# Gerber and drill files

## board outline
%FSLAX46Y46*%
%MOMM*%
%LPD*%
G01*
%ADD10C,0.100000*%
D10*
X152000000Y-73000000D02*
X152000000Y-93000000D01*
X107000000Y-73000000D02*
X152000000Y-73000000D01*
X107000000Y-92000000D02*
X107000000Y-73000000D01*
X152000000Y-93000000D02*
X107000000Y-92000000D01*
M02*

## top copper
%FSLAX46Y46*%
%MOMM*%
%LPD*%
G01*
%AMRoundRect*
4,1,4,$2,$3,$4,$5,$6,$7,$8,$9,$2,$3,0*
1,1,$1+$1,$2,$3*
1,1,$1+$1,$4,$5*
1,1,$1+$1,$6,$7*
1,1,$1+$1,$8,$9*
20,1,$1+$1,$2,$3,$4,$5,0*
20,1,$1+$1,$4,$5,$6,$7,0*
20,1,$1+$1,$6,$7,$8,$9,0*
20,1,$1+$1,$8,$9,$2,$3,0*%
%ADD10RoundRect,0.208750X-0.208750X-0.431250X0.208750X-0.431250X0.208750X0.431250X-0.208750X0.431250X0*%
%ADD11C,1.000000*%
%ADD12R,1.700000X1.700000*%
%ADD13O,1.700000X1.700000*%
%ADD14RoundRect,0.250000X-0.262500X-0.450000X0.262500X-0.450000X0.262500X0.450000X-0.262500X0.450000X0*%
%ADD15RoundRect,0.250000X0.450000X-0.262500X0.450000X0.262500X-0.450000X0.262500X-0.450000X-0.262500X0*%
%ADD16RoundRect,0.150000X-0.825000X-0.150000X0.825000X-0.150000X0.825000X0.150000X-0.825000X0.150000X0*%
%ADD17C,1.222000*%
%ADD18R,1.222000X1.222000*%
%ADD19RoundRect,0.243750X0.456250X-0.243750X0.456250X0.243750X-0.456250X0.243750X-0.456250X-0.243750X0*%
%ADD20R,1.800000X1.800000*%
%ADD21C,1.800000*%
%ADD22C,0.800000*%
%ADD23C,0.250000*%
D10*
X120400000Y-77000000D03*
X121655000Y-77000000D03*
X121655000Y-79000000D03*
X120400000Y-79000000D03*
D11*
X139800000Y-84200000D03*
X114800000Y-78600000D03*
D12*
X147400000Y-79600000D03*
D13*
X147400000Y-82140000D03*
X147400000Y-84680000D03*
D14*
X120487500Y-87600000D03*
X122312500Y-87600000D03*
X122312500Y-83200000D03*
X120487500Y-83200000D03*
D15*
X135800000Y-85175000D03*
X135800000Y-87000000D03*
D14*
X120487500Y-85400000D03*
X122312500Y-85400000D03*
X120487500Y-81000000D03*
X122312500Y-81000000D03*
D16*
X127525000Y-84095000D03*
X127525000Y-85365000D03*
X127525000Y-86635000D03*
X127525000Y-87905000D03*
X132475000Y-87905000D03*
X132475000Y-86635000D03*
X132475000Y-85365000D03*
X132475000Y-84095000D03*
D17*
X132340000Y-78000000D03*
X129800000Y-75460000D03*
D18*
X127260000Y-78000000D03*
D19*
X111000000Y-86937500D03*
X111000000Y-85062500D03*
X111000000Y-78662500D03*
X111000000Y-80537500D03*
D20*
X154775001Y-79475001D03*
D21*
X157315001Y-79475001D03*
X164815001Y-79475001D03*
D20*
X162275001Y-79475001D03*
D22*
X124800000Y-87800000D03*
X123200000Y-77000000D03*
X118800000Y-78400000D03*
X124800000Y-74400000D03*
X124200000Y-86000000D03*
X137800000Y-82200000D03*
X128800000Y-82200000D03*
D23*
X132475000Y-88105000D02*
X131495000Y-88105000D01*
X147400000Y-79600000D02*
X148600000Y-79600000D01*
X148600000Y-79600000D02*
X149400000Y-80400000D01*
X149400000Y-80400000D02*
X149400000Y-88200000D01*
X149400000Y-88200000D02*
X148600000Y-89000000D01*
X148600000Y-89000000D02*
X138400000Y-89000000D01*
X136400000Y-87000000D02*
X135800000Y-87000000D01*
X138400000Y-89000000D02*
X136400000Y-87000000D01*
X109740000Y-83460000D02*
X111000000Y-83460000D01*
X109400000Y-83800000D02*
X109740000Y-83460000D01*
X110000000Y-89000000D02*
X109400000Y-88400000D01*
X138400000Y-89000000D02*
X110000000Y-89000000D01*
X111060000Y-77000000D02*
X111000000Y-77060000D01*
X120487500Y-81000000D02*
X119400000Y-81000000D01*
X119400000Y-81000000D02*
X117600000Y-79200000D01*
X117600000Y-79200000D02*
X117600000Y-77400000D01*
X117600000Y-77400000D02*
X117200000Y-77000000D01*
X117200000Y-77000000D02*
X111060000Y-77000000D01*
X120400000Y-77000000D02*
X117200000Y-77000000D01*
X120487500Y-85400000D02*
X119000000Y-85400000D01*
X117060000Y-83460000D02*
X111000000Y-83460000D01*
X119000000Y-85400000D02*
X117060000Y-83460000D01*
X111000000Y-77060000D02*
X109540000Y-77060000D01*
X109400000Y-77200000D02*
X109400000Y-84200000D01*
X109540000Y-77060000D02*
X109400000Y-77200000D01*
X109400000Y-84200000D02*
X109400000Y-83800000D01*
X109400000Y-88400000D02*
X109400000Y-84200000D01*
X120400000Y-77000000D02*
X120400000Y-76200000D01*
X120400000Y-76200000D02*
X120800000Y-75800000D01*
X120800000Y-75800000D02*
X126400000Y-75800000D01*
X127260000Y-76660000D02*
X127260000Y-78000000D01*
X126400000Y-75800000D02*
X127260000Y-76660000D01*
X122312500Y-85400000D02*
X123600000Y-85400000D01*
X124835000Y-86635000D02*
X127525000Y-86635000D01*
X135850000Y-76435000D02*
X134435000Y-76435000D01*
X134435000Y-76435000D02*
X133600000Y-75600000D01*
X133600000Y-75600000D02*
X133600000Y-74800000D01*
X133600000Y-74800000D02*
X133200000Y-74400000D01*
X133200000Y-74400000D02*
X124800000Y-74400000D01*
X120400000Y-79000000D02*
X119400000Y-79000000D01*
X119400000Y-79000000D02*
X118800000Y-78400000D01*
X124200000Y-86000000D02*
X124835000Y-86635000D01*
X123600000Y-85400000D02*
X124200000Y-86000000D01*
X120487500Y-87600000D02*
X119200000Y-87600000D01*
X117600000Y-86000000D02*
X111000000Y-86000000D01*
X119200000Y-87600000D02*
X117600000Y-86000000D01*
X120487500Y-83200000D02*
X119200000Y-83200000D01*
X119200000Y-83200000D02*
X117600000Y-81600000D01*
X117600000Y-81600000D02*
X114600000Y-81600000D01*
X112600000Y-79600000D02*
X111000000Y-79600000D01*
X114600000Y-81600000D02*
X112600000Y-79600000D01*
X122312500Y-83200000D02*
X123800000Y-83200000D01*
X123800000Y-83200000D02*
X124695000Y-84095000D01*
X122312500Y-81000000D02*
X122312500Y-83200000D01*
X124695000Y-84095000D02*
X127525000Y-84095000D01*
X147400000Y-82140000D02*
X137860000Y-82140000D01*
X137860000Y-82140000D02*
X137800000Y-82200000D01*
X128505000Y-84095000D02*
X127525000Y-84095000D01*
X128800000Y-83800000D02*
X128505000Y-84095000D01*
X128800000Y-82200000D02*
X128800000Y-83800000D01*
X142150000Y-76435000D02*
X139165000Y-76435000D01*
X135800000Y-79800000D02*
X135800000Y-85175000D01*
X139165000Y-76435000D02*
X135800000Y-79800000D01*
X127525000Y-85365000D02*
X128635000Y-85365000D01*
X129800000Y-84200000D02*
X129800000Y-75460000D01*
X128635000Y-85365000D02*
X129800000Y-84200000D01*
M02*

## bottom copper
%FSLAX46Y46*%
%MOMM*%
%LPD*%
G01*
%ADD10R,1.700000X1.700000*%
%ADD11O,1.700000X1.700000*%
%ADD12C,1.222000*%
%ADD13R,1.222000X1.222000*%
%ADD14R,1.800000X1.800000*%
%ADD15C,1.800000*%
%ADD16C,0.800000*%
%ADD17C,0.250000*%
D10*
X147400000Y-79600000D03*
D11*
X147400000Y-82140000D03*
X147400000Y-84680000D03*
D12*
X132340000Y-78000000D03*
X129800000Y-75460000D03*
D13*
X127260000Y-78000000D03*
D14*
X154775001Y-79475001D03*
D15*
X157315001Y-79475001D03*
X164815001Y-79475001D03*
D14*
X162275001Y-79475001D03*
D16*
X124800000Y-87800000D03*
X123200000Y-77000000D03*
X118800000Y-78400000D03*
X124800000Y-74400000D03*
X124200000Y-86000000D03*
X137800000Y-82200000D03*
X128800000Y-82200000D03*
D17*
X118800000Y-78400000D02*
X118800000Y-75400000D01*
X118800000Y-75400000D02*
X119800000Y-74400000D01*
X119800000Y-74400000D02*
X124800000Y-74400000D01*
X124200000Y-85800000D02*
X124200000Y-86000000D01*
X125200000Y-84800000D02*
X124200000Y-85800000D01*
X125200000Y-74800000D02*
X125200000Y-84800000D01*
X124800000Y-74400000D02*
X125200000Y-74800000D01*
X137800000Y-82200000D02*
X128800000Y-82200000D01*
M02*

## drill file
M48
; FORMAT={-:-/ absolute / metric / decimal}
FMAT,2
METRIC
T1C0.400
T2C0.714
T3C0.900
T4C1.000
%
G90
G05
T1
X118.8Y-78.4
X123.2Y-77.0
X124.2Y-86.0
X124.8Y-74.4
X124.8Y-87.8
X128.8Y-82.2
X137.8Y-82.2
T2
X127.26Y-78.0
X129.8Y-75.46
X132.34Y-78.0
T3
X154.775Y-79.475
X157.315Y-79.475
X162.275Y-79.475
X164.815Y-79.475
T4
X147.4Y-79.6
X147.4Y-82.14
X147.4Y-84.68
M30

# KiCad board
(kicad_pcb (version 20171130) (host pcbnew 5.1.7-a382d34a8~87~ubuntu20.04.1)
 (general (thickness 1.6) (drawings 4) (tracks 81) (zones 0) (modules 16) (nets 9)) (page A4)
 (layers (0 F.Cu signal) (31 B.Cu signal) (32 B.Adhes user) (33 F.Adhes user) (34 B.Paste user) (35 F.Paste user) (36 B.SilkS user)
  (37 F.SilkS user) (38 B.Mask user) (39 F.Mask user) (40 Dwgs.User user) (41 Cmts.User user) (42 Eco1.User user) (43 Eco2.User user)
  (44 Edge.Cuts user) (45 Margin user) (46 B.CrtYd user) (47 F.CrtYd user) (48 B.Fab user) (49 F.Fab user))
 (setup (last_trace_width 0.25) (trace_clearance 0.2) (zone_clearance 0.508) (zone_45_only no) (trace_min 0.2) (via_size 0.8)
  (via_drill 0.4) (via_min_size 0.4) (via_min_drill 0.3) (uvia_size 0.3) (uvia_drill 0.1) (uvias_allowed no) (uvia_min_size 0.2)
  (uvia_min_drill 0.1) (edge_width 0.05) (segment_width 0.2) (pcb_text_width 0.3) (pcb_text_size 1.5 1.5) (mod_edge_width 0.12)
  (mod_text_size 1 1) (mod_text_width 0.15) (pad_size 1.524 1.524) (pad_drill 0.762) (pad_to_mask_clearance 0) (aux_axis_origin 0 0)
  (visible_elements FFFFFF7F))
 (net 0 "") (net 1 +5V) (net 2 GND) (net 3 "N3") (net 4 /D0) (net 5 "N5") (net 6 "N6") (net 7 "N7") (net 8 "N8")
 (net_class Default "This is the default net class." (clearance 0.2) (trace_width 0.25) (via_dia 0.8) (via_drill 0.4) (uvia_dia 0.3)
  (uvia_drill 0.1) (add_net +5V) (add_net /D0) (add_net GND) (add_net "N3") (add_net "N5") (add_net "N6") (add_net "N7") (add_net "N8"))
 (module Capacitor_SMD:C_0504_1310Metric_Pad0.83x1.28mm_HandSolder (layer F.Cu) (at 121.0275 77)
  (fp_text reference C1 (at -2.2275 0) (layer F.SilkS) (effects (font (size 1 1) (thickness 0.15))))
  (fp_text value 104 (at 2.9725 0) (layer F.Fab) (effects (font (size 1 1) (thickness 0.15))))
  (pad 1 smd roundrect (at -0.6275 0) (size 0.835 1.28) (layers F.Cu F.Paste F.Mask) (roundrect_rratio 0.25) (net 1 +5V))
  (pad 2 smd roundrect (at 0.6275 0) (size 0.835 1.28) (layers F.Cu F.Paste F.Mask) (roundrect_rratio 0.25) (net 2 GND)))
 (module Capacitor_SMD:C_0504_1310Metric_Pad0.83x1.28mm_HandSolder (layer F.Cu) (at 121.0275 79)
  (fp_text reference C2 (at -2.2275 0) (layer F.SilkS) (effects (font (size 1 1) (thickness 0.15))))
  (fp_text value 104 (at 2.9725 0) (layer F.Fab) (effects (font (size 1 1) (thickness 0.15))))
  (pad 2 smd roundrect (at 0.6275 0) (size 0.835 1.28) (layers F.Cu F.Paste F.Mask) (roundrect_rratio 0.25) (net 2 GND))
  (pad 1 smd roundrect (at -0.6275 0) (size 0.835 1.28) (layers F.Cu F.Paste F.Mask) (roundrect_rratio 0.25) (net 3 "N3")))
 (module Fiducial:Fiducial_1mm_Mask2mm (layer F.Cu) (at 139.8 84.2)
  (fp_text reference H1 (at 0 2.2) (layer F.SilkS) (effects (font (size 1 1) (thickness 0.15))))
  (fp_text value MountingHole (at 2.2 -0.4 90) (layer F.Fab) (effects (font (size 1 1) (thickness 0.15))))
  (pad "" smd circle (at 0 0) (size 1 1) (layers F.Cu F.Mask) (solder_mask_margin 0.5) (clearance 0.5)))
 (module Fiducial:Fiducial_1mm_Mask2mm (layer F.Cu) (at 114.8 78.6)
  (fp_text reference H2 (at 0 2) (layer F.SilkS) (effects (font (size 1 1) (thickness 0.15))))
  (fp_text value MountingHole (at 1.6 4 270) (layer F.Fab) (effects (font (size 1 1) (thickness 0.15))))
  (pad "" smd circle (at 0 0) (size 1 1) (layers F.Cu F.Mask) (solder_mask_margin 0.5) (clearance 0.5)))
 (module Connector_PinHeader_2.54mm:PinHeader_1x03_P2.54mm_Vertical (layer F.Cu) (at 147.4 79.6)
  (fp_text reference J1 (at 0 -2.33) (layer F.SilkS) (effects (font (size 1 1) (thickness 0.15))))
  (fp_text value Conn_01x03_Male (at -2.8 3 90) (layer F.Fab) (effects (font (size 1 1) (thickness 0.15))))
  (pad 1 thru_hole rect (at 0 0) (size 1.7 1.7) (drill 1) (layers *.Cu *.Mask) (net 1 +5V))
  (pad 2 thru_hole oval (at 0 2.54) (size 1.7 1.7) (drill 1) (layers *.Cu *.Mask) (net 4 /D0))
  (pad 3 thru_hole oval (at 0 5.08) (size 1.7 1.7) (drill 1) (layers *.Cu *.Mask) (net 2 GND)))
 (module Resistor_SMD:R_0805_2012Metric (layer F.Cu) (at 121.4 87.6)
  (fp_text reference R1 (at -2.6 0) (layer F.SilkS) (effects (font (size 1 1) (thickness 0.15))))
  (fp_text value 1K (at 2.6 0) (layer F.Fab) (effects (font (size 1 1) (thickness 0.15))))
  (pad 1 smd roundrect (at -0.9125 0) (size 1.025 1.4) (layers F.Cu F.Paste F.Mask) (roundrect_rratio 0.243902) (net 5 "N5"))
  (pad 2 smd roundrect (at 0.9125 0) (size 1.025 1.4) (layers F.Cu F.Paste F.Mask) (roundrect_rratio 0.243902) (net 2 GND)))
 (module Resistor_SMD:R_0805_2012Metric (layer F.Cu) (at 121.4 83.2)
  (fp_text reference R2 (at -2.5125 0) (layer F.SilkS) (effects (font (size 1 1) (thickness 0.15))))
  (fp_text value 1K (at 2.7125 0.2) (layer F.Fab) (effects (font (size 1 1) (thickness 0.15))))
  (pad 2 smd roundrect (at 0.9125 0) (size 1.025 1.4) (layers F.Cu F.Paste F.Mask) (roundrect_rratio 0.243902) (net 4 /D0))
  (pad 1 smd roundrect (at -0.9125 0) (size 1.025 1.4) (layers F.Cu F.Paste F.Mask) (roundrect_rratio 0.243902) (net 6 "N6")))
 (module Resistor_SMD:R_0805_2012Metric (layer F.Cu) (at 135.8 86.0875 90)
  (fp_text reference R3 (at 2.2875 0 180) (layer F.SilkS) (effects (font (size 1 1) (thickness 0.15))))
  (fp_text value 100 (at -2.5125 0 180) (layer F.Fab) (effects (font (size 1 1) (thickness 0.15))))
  (pad 2 smd roundrect (at 0.9125 0 90) (size 1.025 1.4) (layers F.Cu F.Paste F.Mask) (roundrect_rratio 0.243902) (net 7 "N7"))
  (pad 1 smd roundrect (at -0.9125 0 90) (size 1.025 1.4) (layers F.Cu F.Paste F.Mask) (roundrect_rratio 0.243902) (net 1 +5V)))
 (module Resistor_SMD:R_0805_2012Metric (layer F.Cu) (at 121.4 85.4)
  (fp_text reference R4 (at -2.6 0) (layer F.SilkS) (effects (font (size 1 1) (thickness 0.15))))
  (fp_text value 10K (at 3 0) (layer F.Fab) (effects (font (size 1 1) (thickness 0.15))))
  (pad 1 smd roundrect (at -0.9125 0) (size 1.025 1.4) (layers F.Cu F.Paste F.Mask) (roundrect_rratio 0.243902) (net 1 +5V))
  (pad 2 smd roundrect (at 0.9125 0) (size 1.025 1.4) (layers F.Cu F.Paste F.Mask) (roundrect_rratio 0.243902) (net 3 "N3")))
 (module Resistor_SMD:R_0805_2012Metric (layer F.Cu) (at 121.4 81)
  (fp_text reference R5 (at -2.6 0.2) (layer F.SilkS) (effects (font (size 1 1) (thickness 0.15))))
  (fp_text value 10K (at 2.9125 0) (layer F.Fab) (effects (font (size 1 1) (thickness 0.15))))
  (pad 1 smd roundrect (at -0.9125 0) (size 1.025 1.4) (layers F.Cu F.Paste F.Mask) (roundrect_rratio 0.243902) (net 1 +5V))
  (pad 2 smd roundrect (at 0.9125 0) (size 1.025 1.4) (layers F.Cu F.Paste F.Mask) (roundrect_rratio 0.243902) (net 4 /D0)))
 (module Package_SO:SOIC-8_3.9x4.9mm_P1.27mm (layer F.Cu) (at 130 86)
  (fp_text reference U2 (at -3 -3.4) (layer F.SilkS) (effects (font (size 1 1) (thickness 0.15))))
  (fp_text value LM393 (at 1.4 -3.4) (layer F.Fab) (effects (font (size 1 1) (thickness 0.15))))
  (pad 1 smd roundrect (at -2.475 -1.905) (size 1.95 0.6) (layers F.Cu F.Paste F.Mask) (roundrect_rratio 0.25) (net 4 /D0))
  (pad 2 smd roundrect (at -2.475 -0.635) (size 1.95 0.6) (layers F.Cu F.Paste F.Mask) (roundrect_rratio 0.25) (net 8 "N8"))
  (pad 3 smd roundrect (at -2.475 0.635) (size 1.95 0.6) (layers F.Cu F.Paste F.Mask) (roundrect_rratio 0.25) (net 3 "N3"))
  (pad 4 smd roundrect (at -2.475 1.905) (size 1.95 0.6) (layers F.Cu F.Paste F.Mask) (roundrect_rratio 0.25))
  (pad 5 smd roundrect (at 2.475 1.905) (size 1.95 0.6) (layers F.Cu F.Paste F.Mask) (roundrect_rratio 0.25))
  (pad 6 smd roundrect (at 2.475 0.635) (size 1.95 0.6) (layers F.Cu F.Paste F.Mask) (roundrect_rratio 0.25))
  (pad 7 smd roundrect (at 2.475 -0.635) (size 1.95 0.6) (layers F.Cu F.Paste F.Mask) (roundrect_rratio 0.25))
  (pad 8 smd roundrect (at 2.475 -1.905) (size 1.95 0.6) (layers F.Cu F.Paste F.Mask) (roundrect_rratio 0.25)))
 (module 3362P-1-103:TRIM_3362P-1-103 (layer F.Cu) (at 129.8 78)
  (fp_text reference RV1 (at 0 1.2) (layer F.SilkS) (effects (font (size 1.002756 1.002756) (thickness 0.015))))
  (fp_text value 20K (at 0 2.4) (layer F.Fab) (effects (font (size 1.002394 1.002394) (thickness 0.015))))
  (pad 3 thru_hole circle (at 2.54 0) (size 1.222 1.222) (drill 0.714) (layers *.Cu *.Mask) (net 2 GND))
  (pad 2 thru_hole circle (at 0 -2.54) (size 1.222 1.222) (drill 0.714) (layers *.Cu *.Mask) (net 8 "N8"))
  (pad 1 thru_hole rect (at -2.54 0) (size 1.222 1.222) (drill 0.714) (layers *.Cu *.Mask) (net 1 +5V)))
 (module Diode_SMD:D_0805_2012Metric (layer F.Cu) (at 111 86 90)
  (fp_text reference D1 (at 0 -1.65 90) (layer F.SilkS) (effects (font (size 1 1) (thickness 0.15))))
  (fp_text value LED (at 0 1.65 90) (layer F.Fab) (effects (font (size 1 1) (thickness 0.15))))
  (pad 1 smd roundrect (at -0.9375 0 90) (size 0.975 1.4) (layers F.Cu F.Paste F.Mask) (roundrect_rratio 0.25) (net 5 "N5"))
  (pad 2 smd roundrect (at 0.9375 0 90) (size 0.975 1.4) (layers F.Cu F.Paste F.Mask) (roundrect_rratio 0.25) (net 1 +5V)))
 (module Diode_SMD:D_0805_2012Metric (layer F.Cu) (at 111 79.6 90)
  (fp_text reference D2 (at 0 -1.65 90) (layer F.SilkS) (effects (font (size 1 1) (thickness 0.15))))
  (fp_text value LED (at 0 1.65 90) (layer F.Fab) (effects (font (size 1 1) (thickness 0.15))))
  (pad 2 smd roundrect (at 0.9375 0 90) (size 0.975 1.4) (layers F.Cu F.Paste F.Mask) (roundrect_rratio 0.25) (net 1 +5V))
  (pad 1 smd roundrect (at -0.9375 0 90) (size 0.975 1.4) (layers F.Cu F.Paste F.Mask) (roundrect_rratio 0.25) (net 6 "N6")))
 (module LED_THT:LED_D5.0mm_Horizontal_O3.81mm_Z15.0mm (layer F.Cu) (at 154.775001 79.475001)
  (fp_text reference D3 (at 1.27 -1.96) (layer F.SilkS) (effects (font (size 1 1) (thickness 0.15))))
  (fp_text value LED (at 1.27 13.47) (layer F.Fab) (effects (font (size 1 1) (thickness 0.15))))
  (pad 1 thru_hole rect (at 0 0) (size 1.8 1.8) (drill 0.9) (layers *.Cu *.Mask) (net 2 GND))
  (pad 2 thru_hole circle (at 2.54 0) (size 1.8 1.8) (drill 0.9) (layers *.Cu *.Mask) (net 7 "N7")))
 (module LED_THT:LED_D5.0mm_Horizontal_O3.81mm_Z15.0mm (layer F.Cu) (at 162.275001 79.475001)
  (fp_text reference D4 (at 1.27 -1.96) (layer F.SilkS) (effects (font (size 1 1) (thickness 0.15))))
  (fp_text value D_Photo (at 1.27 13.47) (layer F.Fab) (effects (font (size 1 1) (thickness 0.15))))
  (pad 2 thru_hole circle (at 2.54 0) (size 1.8 1.8) (drill 0.9) (layers *.Cu *.Mask) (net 3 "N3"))
  (pad 1 thru_hole rect (at 0 0) (size 1.8 1.8) (drill 0.9) (layers *.Cu *.Mask) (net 2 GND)))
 (gr_line (start 152 73) (end 152 93) (layer Edge.Cuts) (width 0.1))
 (gr_line (start 107 73) (end 152 73) (layer Edge.Cuts) (width 0.1))
 (gr_line (start 107 92) (end 107 73) (layer Edge.Cuts) (width 0.1))
 (gr_line (start 152 93) (end 107 92) (layer Edge.Cuts) (width 0.1))
 (segment (start 132.475 88.105) (end 131.495 88.105) (width 0.25) (layer F.Cu) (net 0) (status 10))
 (segment (start 147.4 79.6) (end 148.6 79.6) (width 0.25) (layer F.Cu) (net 1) (status 10))
 (segment (start 148.6 79.6) (end 149.4 80.4) (width 0.25) (layer F.Cu) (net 1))
 (segment (start 149.4 80.4) (end 149.4 88.2) (width 0.25) (layer F.Cu) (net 1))
 (segment (start 149.4 88.2) (end 148.6 89) (width 0.25) (layer F.Cu) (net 1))
 (segment (start 148.6 89) (end 138.4 89) (width 0.25) (layer F.Cu) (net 1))
 (segment (start 136.4 87) (end 135.8 87) (width 0.25) (layer F.Cu) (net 1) (status 30))
 (segment (start 138.4 89) (end 136.4 87) (width 0.25) (layer F.Cu) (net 1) (status 20))
 (segment (start 109.74 83.46) (end 111 83.46) (width 0.25) (layer F.Cu) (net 1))
 (segment (start 109.4 83.8) (end 109.74 83.46) (width 0.25) (layer F.Cu) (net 1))
 (segment (start 110 89) (end 109.4 88.4) (width 0.25) (layer F.Cu) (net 1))
 (segment (start 138.4 89) (end 110 89) (width 0.25) (layer F.Cu) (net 1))
 (segment (start 111.06 77) (end 111 77.06) (width 0.25) (layer F.Cu) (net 1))
 (segment (start 120.4875 81) (end 119.4 81) (width 0.25) (layer F.Cu) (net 1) (status 10))
 (segment (start 119.4 81) (end 117.6 79.2) (width 0.25) (layer F.Cu) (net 1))
 (segment (start 117.6 79.2) (end 117.6 77.4) (width 0.25) (layer F.Cu) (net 1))
 (segment (start 117.6 77.4) (end 117.2 77) (width 0.25) (layer F.Cu) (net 1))
 (segment (start 117.2 77) (end 111.06 77) (width 0.25) (layer F.Cu) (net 1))
 (segment (start 120.4 77) (end 117.2 77) (width 0.25) (layer F.Cu) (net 1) (status 10))
 (segment (start 120.4875 85.4) (end 119 85.4) (width 0.25) (layer F.Cu) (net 1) (status 10))
 (segment (start 117.06 83.46) (end 111 83.46) (width 0.25) (layer F.Cu) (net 1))
 (segment (start 119 85.4) (end 117.06 83.46) (width 0.25) (layer F.Cu) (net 1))
 (segment (start 111 77.06) (end 109.54 77.06) (width 0.25) (layer F.Cu) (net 1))
 (segment (start 109.4 77.2) (end 109.4 84.2) (width 0.25) (layer F.Cu) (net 1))
 (segment (start 109.54 77.06) (end 109.4 77.2) (width 0.25) (layer F.Cu) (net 1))
 (segment (start 109.4 84.2) (end 109.4 83.8) (width 0.25) (layer F.Cu) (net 1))
 (segment (start 109.4 88.4) (end 109.4 84.2) (width 0.25) (layer F.Cu) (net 1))
 (segment (start 120.4 77) (end 120.4 76.2) (width 0.25) (layer F.Cu) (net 1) (status 10))
 (segment (start 120.4 76.2) (end 120.8 75.8) (width 0.25) (layer F.Cu) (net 1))
 (segment (start 120.8 75.8) (end 126.4 75.8) (width 0.25) (layer F.Cu) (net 1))
 (segment (start 127.26 76.66) (end 127.26 78) (width 0.25) (layer F.Cu) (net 1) (status 20))
 (segment (start 126.4 75.8) (end 127.26 76.66) (width 0.25) (layer F.Cu) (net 1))
 (via (at 124.8 87.8) (size 0.8) (drill 0.4) (layers F.Cu B.Cu) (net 2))
 (via (at 123.2 77) (size 0.8) (drill 0.4) (layers F.Cu B.Cu) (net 2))
 (segment (start 122.3125 85.4) (end 123.6 85.4) (width 0.25) (layer F.Cu) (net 3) (status 10))
 (segment (start 124.835 86.635) (end 127.525 86.635) (width 0.25) (layer F.Cu) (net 3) (status 20))
 (segment (start 135.85 76.435) (end 134.435 76.435) (width 0.25) (layer F.Cu) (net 3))
 (segment (start 134.435 76.435) (end 133.6 75.6) (width 0.25) (layer F.Cu) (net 3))
 (segment (start 133.6 75.6) (end 133.6 74.8) (width 0.25) (layer F.Cu) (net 3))
 (segment (start 133.6 74.8) (end 133.2 74.4) (width 0.25) (layer F.Cu) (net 3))
 (segment (start 133.2 74.4) (end 124.8 74.4) (width 0.25) (layer F.Cu) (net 3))
 (segment (start 120.4 79) (end 119.4 79) (width 0.25) (layer F.Cu) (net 3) (status 10))
 (via (at 118.8 78.4) (size 0.8) (drill 0.4) (layers F.Cu B.Cu) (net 3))
 (segment (start 119.4 79) (end 118.8 78.4) (width 0.25) (layer F.Cu) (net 3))
 (segment (start 118.8 78.4) (end 118.8 75.4) (width 0.25) (layer B.Cu) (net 3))
 (segment (start 118.8 75.4) (end 119.8 74.4) (width 0.25) (layer B.Cu) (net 3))
 (via (at 124.8 74.4) (size 0.8) (drill 0.4) (layers F.Cu B.Cu) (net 3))
 (segment (start 119.8 74.4) (end 124.8 74.4) (width 0.25) (layer B.Cu) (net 3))
 (segment (start 124.2 85.8) (end 124.2 86) (width 0.25) (layer B.Cu) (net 3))
 (segment (start 125.2 84.8) (end 124.2 85.8) (width 0.25) (layer B.Cu) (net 3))
 (segment (start 125.2 74.8) (end 125.2 84.8) (width 0.25) (layer B.Cu) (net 3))
 (segment (start 124.8 74.4) (end 125.2 74.8) (width 0.25) (layer B.Cu) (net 3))
 (via (at 124.2 86) (size 0.8) (drill 0.4) (layers F.Cu B.Cu) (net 3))
 (segment (start 124.2 86) (end 124.835 86.635) (width 0.25) (layer F.Cu) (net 3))
 (segment (start 123.6 85.4) (end 124.2 86) (width 0.25) (layer F.Cu) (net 3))
 (segment (start 120.4875 87.6) (end 119.2 87.6) (width 0.25) (layer F.Cu) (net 5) (status 10))
 (segment (start 117.6 86) (end 111 86) (width 0.25) (layer F.Cu) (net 5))
 (segment (start 119.2 87.6) (end 117.6 86) (width 0.25) (layer F.Cu) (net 5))
 (segment (start 120.4875 83.2) (end 119.2 83.2) (width 0.25) (layer F.Cu) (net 6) (status 10))
 (segment (start 119.2 83.2) (end 117.6 81.6) (width 0.25) (layer F.Cu) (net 6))
 (segment (start 117.6 81.6) (end 114.6 81.6) (width 0.25) (layer F.Cu) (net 6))
 (segment (start 112.6 79.6) (end 111 79.6) (width 0.25) (layer F.Cu) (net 6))
 (segment (start 114.6 81.6) (end 112.6 79.6) (width 0.25) (layer F.Cu) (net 6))
 (segment (start 122.3125 83.2) (end 123.8 83.2) (width 0.25) (layer F.Cu) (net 4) (status 10))
 (segment (start 123.8 83.2) (end 124.695 84.095) (width 0.25) (layer F.Cu) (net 4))
 (segment (start 122.3125 81) (end 122.3125 83.2) (width 0.25) (layer F.Cu) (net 4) (status 30))
 (segment (start 124.695 84.095) (end 127.525 84.095) (width 0.25) (layer F.Cu) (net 4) (status 20))
 (segment (start 147.4 82.14) (end 137.86 82.14) (width 0.25) (layer F.Cu) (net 4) (status 10))
 (via (at 137.8 82.2) (size 0.8) (drill 0.4) (layers F.Cu B.Cu) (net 4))
 (segment (start 137.86 82.14) (end 137.8 82.2) (width 0.25) (layer F.Cu) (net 4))
 (segment (start 137.8 82.2) (end 128.8 82.2) (width 0.25) (layer B.Cu) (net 4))
 (via (at 128.8 82.2) (size 0.8) (drill 0.4) (layers F.Cu B.Cu) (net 4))
 (segment (start 128.505 84.095) (end 127.525 84.095) (width 0.25) (layer F.Cu) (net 4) (status 20))
 (segment (start 128.8 83.8) (end 128.505 84.095) (width 0.25) (layer F.Cu) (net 4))
 (segment (start 128.8 82.2) (end 128.8 83.8) (width 0.25) (layer F.Cu) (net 4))
 (segment (start 142.15 76.435) (end 139.165 76.435) (width 0.25) (layer F.Cu) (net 7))
 (segment (start 135.8 79.8) (end 135.8 85.175) (width 0.25) (layer F.Cu) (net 7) (status 20))
 (segment (start 139.165 76.435) (end 135.8 79.8) (width 0.25) (layer F.Cu) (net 7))
 (segment (start 127.525 85.365) (end 128.635 85.365) (width 0.25) (layer F.Cu) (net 8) (status 10))
 (segment (start 129.8 84.2) (end 129.8 75.46) (width 0.25) (layer F.Cu) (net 8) (status 20))
 (segment (start 128.635 85.365) (end 129.8 84.2) (width 0.25) (layer F.Cu) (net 8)))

